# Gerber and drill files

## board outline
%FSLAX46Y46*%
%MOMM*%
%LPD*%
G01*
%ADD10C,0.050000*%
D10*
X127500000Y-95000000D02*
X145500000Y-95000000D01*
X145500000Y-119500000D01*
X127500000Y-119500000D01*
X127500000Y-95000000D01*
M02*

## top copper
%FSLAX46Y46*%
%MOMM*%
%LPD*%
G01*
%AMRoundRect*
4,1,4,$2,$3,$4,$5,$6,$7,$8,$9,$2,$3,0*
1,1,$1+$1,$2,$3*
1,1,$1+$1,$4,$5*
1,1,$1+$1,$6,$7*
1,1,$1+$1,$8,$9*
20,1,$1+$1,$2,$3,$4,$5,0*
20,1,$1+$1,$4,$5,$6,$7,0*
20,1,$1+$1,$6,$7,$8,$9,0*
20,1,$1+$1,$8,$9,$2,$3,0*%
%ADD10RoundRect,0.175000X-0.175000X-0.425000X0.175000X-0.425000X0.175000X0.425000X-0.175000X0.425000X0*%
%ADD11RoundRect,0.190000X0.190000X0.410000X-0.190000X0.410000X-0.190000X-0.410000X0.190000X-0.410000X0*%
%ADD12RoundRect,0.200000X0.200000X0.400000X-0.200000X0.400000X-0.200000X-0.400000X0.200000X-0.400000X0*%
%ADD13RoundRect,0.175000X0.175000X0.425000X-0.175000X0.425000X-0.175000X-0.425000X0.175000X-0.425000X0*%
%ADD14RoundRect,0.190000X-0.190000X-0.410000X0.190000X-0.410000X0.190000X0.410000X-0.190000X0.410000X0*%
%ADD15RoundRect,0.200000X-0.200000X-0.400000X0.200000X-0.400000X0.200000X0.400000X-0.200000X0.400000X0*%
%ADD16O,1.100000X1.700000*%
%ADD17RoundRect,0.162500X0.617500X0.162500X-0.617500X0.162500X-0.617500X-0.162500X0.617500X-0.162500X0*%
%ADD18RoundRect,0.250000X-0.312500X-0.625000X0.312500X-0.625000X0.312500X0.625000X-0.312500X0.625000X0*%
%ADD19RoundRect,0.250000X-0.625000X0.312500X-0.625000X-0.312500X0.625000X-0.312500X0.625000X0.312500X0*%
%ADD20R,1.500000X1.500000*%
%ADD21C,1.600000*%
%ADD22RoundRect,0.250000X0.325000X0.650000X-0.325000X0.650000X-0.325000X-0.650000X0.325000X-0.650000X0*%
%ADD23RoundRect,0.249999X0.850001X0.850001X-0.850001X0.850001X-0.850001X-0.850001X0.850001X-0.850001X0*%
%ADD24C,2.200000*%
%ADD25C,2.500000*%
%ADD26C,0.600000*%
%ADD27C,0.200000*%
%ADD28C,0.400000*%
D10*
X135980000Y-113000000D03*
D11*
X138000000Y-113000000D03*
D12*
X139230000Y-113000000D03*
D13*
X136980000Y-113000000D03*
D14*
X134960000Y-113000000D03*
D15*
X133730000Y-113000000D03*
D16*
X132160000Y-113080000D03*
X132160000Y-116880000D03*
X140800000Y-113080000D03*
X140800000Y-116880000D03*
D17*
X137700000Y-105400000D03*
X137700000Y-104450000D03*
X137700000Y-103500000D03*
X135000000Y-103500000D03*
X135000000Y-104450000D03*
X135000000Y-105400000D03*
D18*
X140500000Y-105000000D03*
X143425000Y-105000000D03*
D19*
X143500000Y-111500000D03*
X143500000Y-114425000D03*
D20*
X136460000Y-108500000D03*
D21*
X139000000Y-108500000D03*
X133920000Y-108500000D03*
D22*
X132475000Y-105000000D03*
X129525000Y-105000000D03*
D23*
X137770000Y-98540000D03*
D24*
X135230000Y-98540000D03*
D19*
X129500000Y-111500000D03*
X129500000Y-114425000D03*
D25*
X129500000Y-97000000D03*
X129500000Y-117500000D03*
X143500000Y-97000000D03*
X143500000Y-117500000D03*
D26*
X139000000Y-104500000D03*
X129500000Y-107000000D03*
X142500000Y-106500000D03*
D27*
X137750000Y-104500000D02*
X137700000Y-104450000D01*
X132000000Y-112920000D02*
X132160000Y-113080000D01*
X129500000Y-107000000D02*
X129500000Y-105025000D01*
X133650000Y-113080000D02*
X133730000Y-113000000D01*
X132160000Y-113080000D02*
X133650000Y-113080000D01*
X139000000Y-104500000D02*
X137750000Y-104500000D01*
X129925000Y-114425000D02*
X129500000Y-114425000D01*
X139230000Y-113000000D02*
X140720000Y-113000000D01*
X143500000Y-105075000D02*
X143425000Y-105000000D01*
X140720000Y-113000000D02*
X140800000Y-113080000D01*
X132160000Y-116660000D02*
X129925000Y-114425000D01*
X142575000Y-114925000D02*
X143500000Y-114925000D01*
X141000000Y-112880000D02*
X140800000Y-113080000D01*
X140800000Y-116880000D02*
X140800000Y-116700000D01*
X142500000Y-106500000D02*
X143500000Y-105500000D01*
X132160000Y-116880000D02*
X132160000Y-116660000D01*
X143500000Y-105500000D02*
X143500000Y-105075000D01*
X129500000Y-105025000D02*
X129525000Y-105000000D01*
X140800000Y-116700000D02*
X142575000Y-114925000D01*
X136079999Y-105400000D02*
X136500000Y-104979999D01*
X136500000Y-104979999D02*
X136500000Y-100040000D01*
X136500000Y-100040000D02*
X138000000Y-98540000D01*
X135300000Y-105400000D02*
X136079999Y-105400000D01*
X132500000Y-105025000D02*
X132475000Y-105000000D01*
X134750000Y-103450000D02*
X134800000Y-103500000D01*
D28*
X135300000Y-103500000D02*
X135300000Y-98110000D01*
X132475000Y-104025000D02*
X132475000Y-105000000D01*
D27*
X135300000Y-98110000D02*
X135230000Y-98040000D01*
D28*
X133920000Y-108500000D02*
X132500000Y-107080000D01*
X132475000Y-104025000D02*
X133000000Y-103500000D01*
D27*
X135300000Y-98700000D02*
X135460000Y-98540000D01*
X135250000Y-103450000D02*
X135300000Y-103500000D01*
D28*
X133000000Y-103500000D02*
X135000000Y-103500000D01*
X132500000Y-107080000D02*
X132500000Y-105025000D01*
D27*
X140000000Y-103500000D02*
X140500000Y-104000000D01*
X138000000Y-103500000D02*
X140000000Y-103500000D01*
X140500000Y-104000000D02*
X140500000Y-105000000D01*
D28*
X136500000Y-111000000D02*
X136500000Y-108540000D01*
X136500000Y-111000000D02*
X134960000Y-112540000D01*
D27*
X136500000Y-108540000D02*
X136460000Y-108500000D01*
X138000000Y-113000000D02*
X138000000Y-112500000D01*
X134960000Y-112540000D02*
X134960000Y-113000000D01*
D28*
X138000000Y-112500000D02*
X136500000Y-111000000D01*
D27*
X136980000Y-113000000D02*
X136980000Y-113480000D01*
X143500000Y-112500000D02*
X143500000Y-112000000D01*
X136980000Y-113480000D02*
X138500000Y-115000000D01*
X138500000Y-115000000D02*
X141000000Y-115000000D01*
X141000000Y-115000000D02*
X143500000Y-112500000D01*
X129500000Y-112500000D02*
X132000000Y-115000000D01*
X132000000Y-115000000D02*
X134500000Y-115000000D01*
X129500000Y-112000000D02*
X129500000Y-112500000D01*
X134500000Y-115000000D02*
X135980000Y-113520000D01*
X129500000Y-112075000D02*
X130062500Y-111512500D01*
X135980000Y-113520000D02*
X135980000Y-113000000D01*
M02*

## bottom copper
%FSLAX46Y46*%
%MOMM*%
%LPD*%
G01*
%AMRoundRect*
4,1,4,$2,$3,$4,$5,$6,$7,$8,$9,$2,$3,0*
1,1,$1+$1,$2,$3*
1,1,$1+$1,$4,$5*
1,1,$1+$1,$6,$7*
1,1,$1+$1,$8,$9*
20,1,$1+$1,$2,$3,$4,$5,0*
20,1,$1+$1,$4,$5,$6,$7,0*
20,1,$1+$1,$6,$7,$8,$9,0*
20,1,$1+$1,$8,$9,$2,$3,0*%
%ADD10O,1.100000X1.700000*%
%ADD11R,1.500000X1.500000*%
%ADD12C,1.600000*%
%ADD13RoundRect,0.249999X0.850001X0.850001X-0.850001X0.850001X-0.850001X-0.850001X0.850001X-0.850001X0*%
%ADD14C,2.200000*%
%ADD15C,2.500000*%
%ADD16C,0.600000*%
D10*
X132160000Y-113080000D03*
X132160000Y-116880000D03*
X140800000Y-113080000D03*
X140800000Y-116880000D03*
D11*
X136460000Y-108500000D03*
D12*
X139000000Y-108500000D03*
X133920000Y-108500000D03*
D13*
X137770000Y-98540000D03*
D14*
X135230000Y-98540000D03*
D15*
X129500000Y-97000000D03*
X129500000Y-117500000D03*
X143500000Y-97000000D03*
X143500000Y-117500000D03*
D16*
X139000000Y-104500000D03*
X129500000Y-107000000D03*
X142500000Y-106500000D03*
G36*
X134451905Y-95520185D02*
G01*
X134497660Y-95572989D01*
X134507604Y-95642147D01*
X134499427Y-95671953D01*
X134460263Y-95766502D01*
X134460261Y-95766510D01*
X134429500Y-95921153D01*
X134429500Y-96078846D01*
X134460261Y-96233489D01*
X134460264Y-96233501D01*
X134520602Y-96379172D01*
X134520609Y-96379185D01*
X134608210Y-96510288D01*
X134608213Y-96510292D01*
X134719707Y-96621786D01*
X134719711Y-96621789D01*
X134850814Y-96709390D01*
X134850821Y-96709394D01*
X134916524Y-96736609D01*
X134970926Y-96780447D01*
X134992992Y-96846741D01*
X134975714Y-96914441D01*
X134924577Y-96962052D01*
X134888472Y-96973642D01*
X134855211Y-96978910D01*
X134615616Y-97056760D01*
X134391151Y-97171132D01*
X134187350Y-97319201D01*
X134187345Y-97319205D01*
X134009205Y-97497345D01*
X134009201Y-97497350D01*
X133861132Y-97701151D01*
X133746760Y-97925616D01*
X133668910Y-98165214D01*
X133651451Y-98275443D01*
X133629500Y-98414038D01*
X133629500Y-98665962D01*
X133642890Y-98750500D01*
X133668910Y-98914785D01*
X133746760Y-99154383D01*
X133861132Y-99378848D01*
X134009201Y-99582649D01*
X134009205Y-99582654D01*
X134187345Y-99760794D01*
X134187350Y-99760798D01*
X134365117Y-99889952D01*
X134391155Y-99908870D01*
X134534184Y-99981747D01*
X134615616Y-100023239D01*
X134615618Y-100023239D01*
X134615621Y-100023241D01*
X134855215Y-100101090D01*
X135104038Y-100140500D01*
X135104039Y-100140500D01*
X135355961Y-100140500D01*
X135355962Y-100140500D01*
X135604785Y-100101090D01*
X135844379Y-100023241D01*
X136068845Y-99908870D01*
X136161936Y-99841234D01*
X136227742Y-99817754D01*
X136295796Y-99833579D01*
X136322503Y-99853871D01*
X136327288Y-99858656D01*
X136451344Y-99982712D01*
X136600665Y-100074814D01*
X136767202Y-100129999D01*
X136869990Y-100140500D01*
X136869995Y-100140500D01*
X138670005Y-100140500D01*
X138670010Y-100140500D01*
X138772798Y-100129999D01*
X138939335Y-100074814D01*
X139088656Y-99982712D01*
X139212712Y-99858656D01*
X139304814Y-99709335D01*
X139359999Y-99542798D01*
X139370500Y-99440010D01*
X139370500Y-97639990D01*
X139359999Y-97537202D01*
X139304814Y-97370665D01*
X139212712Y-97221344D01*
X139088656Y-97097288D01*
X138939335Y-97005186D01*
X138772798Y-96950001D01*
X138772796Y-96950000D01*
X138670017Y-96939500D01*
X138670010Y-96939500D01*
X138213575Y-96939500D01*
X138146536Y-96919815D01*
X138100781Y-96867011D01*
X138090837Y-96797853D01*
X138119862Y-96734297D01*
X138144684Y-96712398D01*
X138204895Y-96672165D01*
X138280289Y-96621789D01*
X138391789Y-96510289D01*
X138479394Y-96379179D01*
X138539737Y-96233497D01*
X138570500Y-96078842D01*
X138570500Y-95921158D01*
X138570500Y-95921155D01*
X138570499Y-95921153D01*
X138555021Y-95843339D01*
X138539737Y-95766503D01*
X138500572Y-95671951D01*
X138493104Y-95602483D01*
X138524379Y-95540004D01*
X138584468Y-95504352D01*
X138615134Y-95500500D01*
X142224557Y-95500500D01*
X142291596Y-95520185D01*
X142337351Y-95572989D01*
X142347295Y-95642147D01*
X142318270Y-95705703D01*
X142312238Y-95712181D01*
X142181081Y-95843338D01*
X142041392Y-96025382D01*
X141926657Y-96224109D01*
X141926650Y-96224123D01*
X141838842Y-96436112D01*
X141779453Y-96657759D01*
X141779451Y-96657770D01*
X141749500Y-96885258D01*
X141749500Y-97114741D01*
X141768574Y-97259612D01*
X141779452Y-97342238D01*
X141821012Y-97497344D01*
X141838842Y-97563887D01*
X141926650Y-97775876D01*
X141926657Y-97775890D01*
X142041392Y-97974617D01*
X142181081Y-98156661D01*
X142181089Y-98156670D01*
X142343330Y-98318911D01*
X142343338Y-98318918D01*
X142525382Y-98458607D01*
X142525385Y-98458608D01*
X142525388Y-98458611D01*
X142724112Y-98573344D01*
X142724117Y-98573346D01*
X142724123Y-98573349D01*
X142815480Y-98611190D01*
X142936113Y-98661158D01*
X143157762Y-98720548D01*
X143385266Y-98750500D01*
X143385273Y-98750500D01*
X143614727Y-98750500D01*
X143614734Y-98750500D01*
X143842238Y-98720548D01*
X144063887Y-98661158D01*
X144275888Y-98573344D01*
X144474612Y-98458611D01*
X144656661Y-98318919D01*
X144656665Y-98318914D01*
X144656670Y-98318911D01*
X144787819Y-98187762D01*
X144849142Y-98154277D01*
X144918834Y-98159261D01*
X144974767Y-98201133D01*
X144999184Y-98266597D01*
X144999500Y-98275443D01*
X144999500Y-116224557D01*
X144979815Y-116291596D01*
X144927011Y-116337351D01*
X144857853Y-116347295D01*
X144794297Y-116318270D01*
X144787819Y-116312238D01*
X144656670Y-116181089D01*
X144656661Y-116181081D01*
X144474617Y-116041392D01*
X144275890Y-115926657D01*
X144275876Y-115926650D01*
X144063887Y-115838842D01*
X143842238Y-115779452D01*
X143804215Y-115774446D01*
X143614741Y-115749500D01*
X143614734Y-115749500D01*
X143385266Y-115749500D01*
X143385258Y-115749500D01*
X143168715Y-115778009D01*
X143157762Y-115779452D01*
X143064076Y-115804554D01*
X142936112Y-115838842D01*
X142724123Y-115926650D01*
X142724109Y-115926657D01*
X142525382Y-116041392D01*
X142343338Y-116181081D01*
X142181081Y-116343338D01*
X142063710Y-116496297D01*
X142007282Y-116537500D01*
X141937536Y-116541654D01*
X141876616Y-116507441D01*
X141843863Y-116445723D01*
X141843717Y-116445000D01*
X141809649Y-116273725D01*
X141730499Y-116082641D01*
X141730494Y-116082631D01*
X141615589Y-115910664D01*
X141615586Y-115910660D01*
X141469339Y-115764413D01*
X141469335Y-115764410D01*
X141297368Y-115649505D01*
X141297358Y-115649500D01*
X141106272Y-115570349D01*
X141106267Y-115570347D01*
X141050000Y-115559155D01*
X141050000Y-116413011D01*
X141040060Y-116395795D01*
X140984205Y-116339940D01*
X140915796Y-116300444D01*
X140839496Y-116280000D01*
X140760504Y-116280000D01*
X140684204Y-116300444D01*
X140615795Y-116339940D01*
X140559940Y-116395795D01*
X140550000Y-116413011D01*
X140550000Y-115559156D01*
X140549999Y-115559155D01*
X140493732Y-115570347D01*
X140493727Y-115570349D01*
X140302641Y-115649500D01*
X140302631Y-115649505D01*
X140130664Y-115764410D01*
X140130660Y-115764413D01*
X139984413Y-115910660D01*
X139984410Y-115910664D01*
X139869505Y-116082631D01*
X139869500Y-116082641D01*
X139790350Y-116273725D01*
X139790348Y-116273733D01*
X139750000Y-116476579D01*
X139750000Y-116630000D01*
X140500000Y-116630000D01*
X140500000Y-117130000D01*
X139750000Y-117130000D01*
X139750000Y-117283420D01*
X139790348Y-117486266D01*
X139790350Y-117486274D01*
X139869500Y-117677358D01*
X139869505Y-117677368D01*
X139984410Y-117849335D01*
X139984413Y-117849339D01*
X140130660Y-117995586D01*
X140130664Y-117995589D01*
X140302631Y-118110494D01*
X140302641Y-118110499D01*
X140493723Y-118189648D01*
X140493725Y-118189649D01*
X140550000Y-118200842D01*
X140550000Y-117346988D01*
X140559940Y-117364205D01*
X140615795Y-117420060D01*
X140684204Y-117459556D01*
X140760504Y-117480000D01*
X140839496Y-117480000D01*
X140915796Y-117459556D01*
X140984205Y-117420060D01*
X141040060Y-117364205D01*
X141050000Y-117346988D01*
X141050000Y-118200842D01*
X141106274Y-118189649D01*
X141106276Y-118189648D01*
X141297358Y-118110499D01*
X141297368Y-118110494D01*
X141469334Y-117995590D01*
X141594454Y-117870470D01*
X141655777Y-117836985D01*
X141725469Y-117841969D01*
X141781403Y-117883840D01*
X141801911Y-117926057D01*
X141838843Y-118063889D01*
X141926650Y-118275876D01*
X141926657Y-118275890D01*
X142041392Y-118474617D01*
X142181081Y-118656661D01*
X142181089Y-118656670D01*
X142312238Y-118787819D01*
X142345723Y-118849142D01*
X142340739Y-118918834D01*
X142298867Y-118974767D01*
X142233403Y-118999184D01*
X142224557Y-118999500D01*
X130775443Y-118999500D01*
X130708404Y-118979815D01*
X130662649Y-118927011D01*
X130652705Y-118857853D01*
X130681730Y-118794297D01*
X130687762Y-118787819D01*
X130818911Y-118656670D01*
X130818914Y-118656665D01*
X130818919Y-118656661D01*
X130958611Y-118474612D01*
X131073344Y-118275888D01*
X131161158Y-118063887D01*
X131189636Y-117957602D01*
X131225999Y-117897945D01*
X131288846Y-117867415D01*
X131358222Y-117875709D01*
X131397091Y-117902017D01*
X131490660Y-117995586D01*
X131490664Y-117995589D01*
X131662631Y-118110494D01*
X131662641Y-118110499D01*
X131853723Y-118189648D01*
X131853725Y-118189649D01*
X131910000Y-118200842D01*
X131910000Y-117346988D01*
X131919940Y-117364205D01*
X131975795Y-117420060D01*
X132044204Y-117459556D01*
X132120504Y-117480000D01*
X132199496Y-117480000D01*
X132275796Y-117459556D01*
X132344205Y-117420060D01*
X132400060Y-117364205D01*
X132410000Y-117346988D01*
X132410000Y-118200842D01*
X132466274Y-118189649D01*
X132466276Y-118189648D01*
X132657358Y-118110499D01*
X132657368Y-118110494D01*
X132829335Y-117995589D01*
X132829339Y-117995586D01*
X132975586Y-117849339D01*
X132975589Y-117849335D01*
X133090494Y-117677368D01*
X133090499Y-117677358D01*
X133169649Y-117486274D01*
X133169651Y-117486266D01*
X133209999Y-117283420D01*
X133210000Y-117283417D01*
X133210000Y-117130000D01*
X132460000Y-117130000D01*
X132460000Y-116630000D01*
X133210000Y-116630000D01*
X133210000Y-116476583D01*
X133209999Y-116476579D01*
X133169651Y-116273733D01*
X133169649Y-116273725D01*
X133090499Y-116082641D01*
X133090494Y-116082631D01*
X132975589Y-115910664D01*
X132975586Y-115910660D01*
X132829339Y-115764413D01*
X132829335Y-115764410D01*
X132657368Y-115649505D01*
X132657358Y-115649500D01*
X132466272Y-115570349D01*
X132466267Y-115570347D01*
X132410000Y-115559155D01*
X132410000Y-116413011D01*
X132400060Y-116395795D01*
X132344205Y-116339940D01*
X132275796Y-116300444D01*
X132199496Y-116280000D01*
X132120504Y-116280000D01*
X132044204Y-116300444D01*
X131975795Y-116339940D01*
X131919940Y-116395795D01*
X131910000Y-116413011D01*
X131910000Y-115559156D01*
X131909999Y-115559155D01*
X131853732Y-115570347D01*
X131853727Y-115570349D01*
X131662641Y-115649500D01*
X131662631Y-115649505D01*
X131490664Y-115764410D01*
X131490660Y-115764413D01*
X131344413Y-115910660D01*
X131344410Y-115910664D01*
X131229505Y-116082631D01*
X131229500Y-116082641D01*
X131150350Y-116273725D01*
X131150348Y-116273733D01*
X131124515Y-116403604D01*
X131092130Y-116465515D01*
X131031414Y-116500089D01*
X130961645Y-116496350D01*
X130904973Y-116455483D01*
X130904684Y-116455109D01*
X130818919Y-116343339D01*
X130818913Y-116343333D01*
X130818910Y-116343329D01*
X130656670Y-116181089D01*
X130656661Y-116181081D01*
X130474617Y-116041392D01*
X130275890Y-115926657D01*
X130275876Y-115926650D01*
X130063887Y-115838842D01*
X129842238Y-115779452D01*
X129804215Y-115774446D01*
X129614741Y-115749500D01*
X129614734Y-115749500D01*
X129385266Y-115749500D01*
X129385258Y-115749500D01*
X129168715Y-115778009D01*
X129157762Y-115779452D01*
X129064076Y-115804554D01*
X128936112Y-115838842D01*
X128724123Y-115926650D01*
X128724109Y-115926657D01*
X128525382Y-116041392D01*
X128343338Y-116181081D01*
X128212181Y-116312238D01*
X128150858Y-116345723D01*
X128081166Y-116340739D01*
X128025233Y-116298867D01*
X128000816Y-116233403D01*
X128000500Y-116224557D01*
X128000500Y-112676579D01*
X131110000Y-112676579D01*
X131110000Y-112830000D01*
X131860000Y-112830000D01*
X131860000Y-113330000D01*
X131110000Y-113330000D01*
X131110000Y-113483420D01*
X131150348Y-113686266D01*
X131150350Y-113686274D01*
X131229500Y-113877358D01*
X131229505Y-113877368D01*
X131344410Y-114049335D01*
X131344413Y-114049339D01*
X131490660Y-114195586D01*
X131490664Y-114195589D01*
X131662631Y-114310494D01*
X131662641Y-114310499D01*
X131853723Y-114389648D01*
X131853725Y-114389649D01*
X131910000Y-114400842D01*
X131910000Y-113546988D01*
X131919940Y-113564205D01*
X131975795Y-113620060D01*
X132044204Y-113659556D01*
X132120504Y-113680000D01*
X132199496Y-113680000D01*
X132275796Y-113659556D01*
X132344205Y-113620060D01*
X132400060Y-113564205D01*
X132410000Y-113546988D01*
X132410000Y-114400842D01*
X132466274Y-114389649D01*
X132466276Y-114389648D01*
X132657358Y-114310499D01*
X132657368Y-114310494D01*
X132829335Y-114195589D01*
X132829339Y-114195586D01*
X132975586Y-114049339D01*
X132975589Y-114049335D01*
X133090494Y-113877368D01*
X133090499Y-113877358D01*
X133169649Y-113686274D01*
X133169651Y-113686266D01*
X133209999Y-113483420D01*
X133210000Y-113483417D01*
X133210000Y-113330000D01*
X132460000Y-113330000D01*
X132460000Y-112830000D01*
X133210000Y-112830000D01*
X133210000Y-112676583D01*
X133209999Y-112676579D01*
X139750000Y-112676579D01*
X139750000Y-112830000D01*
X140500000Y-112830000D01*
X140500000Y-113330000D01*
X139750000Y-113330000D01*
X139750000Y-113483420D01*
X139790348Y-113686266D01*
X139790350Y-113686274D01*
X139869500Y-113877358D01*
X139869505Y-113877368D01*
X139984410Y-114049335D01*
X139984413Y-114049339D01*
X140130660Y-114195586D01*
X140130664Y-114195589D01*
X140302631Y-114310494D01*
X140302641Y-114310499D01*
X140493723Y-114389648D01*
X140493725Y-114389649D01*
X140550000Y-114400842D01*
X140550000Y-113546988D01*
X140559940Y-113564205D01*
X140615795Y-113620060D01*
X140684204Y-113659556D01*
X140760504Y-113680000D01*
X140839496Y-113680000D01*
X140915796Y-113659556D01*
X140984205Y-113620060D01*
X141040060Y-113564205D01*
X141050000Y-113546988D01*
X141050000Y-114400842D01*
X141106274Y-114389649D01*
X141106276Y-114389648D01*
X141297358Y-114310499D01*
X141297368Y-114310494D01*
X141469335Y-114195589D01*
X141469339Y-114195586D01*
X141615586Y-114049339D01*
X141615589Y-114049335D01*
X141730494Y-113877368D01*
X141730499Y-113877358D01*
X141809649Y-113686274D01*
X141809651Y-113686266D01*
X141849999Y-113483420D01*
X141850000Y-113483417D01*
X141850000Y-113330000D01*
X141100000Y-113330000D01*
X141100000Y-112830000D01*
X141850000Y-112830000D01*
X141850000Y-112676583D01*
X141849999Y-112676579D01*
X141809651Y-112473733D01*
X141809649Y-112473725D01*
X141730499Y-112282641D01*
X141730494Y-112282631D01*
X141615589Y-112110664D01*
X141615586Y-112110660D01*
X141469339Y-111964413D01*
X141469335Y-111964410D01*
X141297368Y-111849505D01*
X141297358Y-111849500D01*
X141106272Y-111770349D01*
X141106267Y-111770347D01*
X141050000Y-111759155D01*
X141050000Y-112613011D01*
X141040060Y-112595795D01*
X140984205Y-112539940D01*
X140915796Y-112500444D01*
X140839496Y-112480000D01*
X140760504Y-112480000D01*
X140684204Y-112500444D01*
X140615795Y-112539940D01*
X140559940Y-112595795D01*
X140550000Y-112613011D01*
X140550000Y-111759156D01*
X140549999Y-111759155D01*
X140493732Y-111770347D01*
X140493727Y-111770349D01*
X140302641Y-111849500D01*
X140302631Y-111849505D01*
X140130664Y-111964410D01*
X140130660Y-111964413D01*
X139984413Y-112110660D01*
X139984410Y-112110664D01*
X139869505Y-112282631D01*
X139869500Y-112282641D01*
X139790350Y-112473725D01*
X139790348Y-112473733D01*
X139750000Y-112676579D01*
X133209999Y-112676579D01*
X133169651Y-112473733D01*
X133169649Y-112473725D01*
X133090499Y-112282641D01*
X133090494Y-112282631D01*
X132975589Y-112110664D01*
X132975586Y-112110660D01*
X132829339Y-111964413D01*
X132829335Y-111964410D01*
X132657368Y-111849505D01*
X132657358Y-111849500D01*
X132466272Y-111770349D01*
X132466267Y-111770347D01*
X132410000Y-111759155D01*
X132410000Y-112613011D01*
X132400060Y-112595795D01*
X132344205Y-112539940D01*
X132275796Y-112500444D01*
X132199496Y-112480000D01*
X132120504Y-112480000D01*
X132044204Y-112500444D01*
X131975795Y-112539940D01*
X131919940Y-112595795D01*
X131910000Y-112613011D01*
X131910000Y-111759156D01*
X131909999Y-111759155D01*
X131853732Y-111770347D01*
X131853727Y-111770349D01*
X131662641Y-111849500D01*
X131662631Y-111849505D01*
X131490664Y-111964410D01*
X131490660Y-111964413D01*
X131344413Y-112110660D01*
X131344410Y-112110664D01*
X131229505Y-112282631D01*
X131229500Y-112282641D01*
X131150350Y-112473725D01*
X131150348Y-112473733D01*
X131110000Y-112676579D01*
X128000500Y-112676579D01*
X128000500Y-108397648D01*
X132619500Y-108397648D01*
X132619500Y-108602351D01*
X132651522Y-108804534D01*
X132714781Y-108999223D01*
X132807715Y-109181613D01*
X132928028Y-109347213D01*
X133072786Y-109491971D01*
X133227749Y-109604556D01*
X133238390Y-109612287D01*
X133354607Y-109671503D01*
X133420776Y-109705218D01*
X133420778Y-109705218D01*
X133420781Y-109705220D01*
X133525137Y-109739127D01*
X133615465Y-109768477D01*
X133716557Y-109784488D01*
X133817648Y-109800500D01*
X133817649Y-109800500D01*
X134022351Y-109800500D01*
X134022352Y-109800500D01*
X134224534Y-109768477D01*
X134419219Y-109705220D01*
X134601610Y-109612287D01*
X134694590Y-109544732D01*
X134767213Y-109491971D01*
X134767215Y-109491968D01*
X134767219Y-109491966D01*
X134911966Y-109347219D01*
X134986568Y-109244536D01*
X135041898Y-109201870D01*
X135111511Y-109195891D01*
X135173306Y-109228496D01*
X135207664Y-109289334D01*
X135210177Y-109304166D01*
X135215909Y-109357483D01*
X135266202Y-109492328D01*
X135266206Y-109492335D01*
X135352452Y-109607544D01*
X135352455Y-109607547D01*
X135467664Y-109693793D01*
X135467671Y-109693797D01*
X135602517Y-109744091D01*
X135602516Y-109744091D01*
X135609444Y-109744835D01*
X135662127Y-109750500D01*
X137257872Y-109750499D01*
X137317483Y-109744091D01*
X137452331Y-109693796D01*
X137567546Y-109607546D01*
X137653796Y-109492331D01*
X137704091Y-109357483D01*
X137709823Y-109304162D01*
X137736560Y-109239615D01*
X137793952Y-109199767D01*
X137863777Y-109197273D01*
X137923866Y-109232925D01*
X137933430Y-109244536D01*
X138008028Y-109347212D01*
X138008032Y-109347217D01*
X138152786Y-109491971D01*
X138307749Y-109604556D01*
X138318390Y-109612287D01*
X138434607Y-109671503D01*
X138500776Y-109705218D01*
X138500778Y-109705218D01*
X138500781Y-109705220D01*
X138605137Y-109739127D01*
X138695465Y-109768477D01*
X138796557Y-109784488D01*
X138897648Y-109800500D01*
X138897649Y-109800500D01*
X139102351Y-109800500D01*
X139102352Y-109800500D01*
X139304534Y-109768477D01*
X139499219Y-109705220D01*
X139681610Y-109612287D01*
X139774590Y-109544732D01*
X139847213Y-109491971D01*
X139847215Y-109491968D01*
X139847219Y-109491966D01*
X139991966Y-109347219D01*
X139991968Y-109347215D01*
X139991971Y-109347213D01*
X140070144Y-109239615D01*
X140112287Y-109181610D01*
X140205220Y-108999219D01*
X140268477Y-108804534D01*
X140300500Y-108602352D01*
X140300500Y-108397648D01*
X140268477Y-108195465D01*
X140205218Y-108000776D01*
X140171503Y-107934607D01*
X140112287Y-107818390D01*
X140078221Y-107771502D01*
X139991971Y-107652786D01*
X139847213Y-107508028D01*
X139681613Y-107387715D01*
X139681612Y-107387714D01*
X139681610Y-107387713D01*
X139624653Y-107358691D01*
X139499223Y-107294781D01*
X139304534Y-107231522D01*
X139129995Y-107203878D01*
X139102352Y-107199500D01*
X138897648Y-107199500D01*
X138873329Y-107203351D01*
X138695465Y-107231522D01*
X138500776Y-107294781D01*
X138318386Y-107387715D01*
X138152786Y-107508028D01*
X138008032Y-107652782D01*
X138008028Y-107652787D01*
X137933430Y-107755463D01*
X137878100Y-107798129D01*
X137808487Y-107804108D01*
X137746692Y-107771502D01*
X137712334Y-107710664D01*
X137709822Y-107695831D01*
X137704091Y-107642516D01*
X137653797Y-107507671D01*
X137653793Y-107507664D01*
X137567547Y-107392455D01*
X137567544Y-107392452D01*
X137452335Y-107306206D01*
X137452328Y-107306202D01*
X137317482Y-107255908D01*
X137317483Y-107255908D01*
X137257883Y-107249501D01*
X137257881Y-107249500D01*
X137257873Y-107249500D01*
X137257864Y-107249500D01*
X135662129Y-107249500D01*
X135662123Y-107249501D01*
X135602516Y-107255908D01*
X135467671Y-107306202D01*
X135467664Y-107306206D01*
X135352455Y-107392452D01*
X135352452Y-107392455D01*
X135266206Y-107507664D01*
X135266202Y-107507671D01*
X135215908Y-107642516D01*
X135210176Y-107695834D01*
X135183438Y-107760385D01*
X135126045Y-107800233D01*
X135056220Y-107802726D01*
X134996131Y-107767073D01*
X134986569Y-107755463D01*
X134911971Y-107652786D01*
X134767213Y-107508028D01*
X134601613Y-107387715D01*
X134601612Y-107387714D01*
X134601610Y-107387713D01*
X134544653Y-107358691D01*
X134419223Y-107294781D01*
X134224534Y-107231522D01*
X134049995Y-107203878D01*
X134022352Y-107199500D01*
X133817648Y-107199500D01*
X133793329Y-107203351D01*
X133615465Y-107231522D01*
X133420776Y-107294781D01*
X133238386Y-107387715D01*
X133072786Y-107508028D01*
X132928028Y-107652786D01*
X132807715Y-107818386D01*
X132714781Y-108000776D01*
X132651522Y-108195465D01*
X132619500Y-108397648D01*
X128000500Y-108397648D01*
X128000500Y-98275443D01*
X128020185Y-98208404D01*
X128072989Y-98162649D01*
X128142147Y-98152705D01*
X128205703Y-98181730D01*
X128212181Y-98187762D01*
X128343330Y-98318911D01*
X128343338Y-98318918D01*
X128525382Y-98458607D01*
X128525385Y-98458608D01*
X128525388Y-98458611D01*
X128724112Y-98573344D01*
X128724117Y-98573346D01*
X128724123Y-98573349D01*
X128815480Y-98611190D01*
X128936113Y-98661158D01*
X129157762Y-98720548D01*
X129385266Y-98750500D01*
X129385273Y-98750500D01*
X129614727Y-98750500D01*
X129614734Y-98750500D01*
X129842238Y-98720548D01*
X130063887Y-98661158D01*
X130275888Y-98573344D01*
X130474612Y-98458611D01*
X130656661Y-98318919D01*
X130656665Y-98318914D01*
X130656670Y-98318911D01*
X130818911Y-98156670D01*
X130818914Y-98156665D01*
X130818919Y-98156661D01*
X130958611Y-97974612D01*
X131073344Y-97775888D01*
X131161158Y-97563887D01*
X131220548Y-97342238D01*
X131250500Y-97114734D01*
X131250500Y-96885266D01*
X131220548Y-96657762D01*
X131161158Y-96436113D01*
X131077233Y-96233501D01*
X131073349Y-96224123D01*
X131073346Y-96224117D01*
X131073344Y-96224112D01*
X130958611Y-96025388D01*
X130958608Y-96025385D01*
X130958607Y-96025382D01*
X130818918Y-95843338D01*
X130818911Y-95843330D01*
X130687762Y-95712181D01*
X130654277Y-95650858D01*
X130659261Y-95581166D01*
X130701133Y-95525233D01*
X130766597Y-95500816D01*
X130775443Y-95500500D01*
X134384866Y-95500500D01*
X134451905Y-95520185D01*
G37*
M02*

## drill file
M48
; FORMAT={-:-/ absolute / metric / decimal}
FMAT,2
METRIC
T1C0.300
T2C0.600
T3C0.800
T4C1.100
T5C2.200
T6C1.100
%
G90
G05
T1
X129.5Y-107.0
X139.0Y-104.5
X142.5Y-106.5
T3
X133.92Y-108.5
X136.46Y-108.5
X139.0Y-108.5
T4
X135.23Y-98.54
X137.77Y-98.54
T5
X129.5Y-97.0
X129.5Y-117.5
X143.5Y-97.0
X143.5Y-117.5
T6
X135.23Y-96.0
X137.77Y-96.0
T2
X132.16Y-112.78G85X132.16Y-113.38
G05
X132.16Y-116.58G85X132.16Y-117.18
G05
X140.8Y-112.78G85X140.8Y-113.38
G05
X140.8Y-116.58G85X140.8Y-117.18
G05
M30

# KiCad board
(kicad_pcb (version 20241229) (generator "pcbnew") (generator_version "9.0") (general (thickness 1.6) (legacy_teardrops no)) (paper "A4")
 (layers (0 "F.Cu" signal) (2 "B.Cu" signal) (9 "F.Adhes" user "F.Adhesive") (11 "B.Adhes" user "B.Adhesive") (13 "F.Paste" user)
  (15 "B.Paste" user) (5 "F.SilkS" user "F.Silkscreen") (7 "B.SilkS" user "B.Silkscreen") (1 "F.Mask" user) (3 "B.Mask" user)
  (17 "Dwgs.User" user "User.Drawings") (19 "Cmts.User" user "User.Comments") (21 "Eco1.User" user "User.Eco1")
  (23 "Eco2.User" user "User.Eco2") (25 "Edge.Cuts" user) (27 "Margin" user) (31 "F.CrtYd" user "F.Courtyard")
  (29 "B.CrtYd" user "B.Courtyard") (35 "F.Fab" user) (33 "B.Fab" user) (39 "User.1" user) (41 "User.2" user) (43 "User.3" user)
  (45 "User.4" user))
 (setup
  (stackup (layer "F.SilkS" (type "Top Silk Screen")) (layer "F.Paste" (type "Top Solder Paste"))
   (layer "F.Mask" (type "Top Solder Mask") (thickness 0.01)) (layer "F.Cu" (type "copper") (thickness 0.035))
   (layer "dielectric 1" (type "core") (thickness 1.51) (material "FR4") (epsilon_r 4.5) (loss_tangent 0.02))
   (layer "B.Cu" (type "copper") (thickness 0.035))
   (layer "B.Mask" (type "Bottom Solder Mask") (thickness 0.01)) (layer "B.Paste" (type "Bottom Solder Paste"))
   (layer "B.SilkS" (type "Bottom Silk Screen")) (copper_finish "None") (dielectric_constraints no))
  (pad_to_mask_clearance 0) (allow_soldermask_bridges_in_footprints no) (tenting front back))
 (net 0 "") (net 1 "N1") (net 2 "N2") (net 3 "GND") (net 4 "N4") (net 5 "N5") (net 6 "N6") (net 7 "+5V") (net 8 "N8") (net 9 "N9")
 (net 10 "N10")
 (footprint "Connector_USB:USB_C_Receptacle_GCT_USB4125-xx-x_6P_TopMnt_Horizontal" (layer "F.Cu") (at 136.48 116.08)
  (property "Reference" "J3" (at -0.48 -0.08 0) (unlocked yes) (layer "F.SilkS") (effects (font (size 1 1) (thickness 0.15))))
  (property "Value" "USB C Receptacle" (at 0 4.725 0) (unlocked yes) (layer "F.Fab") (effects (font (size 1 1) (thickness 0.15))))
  (pad "A5" smd roundrect (at -0.5 -3.08) (size 0.7 1.2) (layers "F.Cu" "F.Mask" "F.Paste") (roundrect_rratio 0.25) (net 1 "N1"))
  (pad "A9" smd roundrect (at 1.52 -3.08 180) (size 0.76 1.2) (layers "F.Cu" "F.Mask" "F.Paste") (roundrect_rratio 0.25) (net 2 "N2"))
  (pad "A12" smd roundrect (at 2.75 -3.08 180) (size 0.8 1.2) (layers "F.Cu" "F.Mask" "F.Paste") (roundrect_rratio 0.25) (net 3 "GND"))
  (pad "B5" smd roundrect (at 0.5 -3.08 180) (size 0.7 1.2) (layers "F.Cu" "F.Mask" "F.Paste") (roundrect_rratio 0.25) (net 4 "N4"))
  (pad "B9" smd roundrect (at -1.52 -3.08) (size 0.76 1.2) (layers "F.Cu" "F.Mask" "F.Paste") (roundrect_rratio 0.25) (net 2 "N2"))
  (pad "B12" smd roundrect (at -2.75 -3.08) (size 0.8 1.2) (layers "F.Cu" "F.Mask" "F.Paste") (roundrect_rratio 0.25) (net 3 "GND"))
  (pad "S1" thru_hole oval (at -4.32 -3) (size 1.1 1.7) (drill oval 0.6 1.2) (layers "*.Cu" "*.Mask" "F.Paste") (remove_unused_layers no)
   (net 3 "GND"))
  (pad "S1" thru_hole oval (at -4.32 0.8) (size 1.1 1.7) (drill oval 0.6 1.2) (layers "*.Cu" "*.Mask" "F.Paste") (remove_unused_layers no)
   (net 3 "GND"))
  (pad "S1" thru_hole oval (at 4.32 -3) (size 1.1 1.7) (drill oval 0.6 1.2) (layers "*.Cu" "*.Mask" "F.Paste") (remove_unused_layers no)
   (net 3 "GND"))
  (pad "S1" thru_hole oval (at 4.32 0.8) (size 1.1 1.7) (drill oval 0.6 1.2) (layers "*.Cu" "*.Mask" "F.Paste") (remove_unused_layers no)
   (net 3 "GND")))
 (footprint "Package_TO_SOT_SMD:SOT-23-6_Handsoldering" (layer "F.Cu") (at 136.35 104.45 180)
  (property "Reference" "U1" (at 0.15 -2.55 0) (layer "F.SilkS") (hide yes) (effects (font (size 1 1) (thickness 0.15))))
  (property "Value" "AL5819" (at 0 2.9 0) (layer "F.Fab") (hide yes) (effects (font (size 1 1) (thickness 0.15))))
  (pad "1" smd roundrect (at -1.35 -0.95 180) (size 1.56 0.65) (layers "F.Cu" "F.Mask" "F.Paste") (roundrect_rratio 0.25) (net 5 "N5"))
  (pad "2" smd roundrect (at -1.35 0 180) (size 1.56 0.65) (layers "F.Cu" "F.Mask" "F.Paste") (roundrect_rratio 0.25) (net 3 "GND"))
  (pad "3" smd roundrect (at -1.35 0.95 180) (size 1.56 0.65) (layers "F.Cu" "F.Mask" "F.Paste") (roundrect_rratio 0.25) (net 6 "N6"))
  (pad "4" smd roundrect (at 1.35 0.95 180) (size 1.56 0.65) (layers "F.Cu" "F.Mask" "F.Paste") (roundrect_rratio 0.25) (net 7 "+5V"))
  (pad "5" smd roundrect (at 1.35 0 180) (size 1.56 0.65) (layers "F.Cu" "F.Mask" "F.Paste") (roundrect_rratio 0.25) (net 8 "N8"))
  (pad "6" smd roundrect (at 1.35 -0.95 180) (size 1.56 0.65) (layers "F.Cu" "F.Mask" "F.Paste") (roundrect_rratio 0.25) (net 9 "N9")))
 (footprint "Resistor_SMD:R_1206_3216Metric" (layer "F.Cu") (at 141.9625 105)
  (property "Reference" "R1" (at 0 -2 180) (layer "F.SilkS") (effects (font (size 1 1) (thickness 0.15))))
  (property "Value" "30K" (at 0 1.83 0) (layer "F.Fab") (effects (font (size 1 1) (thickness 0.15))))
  (pad "1" smd roundrect (at -1.4625 0) (size 1.125 1.75) (layers "F.Cu" "F.Mask" "F.Paste") (roundrect_rratio 0.222222) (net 6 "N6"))
  (pad "2" smd roundrect (at 1.4625 0) (size 1.125 1.75) (layers "F.Cu" "F.Mask" "F.Paste") (roundrect_rratio 0.222222) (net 3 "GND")))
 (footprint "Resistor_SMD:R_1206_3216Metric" (layer "F.Cu") (at 143.5 112.9625 -90)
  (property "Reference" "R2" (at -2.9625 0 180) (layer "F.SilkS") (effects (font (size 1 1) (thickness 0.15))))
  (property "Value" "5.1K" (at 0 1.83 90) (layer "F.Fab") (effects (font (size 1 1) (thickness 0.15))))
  (pad "1" smd roundrect (at -1.4625 0 270) (size 1.125 1.75) (layers "F.Cu" "F.Mask" "F.Paste") (roundrect_rratio 0.222222) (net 4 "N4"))
  (pad "2" smd roundrect (at 1.4625 0 270) (size 1.125 1.75) (layers "F.Cu" "F.Mask" "F.Paste") (roundrect_rratio 0.222222) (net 3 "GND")))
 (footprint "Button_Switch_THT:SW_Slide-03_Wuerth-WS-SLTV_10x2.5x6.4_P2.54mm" (layer "F.Cu") (at 136.46 108.5 180)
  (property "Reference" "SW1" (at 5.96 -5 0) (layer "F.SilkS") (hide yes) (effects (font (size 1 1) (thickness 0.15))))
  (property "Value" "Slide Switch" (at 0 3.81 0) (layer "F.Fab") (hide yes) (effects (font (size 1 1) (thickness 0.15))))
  (pad "1" thru_hole rect (at 0 0 180) (size 1.5 1.5) (drill 0.8) (layers "*.Cu" "*.Mask") (remove_unused_layers no) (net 2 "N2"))
  (pad "2" thru_hole circle (at -2.54 0 180) (size 1.6 1.6) (drill 0.8) (layers "*.Cu" "*.Mask") (remove_unused_layers no) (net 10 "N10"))
  (pad "3" thru_hole circle (at 2.54 0 180) (size 1.6 1.6) (drill 0.8) (layers "*.Cu" "*.Mask") (remove_unused_layers no) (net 7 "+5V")))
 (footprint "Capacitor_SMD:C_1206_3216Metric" (layer "F.Cu") (at 131 105 180)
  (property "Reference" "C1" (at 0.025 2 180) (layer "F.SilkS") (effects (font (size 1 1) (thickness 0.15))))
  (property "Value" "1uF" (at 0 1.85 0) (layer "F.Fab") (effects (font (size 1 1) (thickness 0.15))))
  (pad "1" smd roundrect (at -1.475 0 180) (size 1.15 1.8) (layers "F.Cu" "F.Mask" "F.Paste") (roundrect_rratio 0.217391) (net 7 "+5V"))
  (pad "2" smd roundrect (at 1.475 0 180) (size 1.15 1.8) (layers "F.Cu" "F.Mask" "F.Paste") (roundrect_rratio 0.217391) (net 3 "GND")))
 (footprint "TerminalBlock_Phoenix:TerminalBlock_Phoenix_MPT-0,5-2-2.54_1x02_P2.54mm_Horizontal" (layer "F.Cu") (at 137.77 98.54 180)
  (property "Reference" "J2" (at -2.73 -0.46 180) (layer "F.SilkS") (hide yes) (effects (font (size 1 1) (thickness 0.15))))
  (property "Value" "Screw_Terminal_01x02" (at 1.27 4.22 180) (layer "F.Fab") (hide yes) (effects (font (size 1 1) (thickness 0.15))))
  (pad "" np_thru_hole circle (at 0 2.54 180) (size 1.1 1.1) (drill 1.1) (layers "*.Cu" "*.Mask"))
  (pad "" np_thru_hole circle (at 2.54 2.54 180) (size 1.1 1.1) (drill 1.1) (layers "*.Cu" "*.Mask"))
  (pad "1" thru_hole roundrect (at 0 0 180) (size 2.2 2.2) (drill 1.1) (layers "*.Cu" "*.Mask") (remove_unused_layers no)
   (roundrect_rratio 0.113636) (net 9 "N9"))
  (pad "2" thru_hole circle (at 2.54 0 180) (size 2.2 2.2) (drill 1.1) (layers "*.Cu" "*.Mask") (remove_unused_layers no) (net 7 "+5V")))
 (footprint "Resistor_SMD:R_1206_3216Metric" (layer "F.Cu") (at 129.5 112.9625 -90)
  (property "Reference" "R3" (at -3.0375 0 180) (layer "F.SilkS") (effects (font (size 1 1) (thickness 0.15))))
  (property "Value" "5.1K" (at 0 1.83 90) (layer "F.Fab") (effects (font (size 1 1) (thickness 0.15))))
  (pad "1" smd roundrect (at -1.4625 0 270) (size 1.125 1.75) (layers "F.Cu" "F.Mask" "F.Paste") (roundrect_rratio 0.222222) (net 1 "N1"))
  (pad "2" smd roundrect (at 1.4625 0 270) (size 1.125 1.75) (layers "F.Cu" "F.Mask" "F.Paste") (roundrect_rratio 0.222222) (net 3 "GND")))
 (gr_rect (start 127.5 95) (end 145.5 119.5) (stroke (width 0.05) (type default)) (fill no) (layer "Edge.Cuts"))
 (via (at 129.5 97) (size 2.5) (drill 2.2) (layers "F.Cu" "B.Cu") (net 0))
 (via (at 129.5 117.5) (size 2.5) (drill 2.2) (layers "F.Cu" "B.Cu") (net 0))
 (via (at 143.5 97) (size 2.5) (drill 2.2) (layers "F.Cu" "B.Cu") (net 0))
 (via (at 143.5 117.5) (size 2.5) (drill 2.2) (layers "F.Cu" "B.Cu") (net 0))
 (segment (start 137.75 104.5) (end 137.7 104.45) (width 0.2) (layer "F.Cu") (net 3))
 (segment (start 132 112.92) (end 132.16 113.08) (width 0.2) (layer "F.Cu") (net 3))
 (segment (start 129.5 107) (end 129.5 105.025) (width 0.2) (layer "F.Cu") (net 3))
 (segment (start 133.65 113.08) (end 133.73 113) (width 0.2) (layer "F.Cu") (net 3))
 (segment (start 132.16 113.08) (end 133.65 113.08) (width 0.2) (layer "F.Cu") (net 3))
 (segment (start 139 104.5) (end 137.75 104.5) (width 0.2) (layer "F.Cu") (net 3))
 (segment (start 129.925 114.425) (end 129.5 114.425) (width 0.2) (layer "F.Cu") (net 3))
 (segment (start 139.23 113) (end 140.72 113) (width 0.2) (layer "F.Cu") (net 3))
 (segment (start 143.5 105.075) (end 143.425 105) (width 0.2) (layer "F.Cu") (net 3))
 (segment (start 140.72 113) (end 140.8 113.08) (width 0.2) (layer "F.Cu") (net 3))
 (segment (start 132.16 116.66) (end 129.925 114.425) (width 0.2) (layer "F.Cu") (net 3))
 (segment (start 142.575 114.925) (end 143.5 114.925) (width 0.2) (layer "F.Cu") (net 3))
 (segment (start 141 112.88) (end 140.8 113.08) (width 0.2) (layer "F.Cu") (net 3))
 (segment (start 140.8 116.88) (end 140.8 116.7) (width 0.2) (layer "F.Cu") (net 3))
 (segment (start 142.5 106.5) (end 143.5 105.5) (width 0.2) (layer "F.Cu") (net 3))
 (segment (start 132.16 116.88) (end 132.16 116.66) (width 0.2) (layer "F.Cu") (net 3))
 (segment (start 143.5 105.5) (end 143.5 105.075) (width 0.2) (layer "F.Cu") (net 3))
 (segment (start 129.5 105.025) (end 129.525 105) (width 0.2) (layer "F.Cu") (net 3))
 (segment (start 140.8 116.7) (end 142.575 114.925) (width 0.2) (layer "F.Cu") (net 3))
 (via (at 139 104.5) (size 0.6) (drill 0.3) (layers "F.Cu" "B.Cu") (free yes) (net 3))
 (via (at 129.5 107) (size 0.6) (drill 0.3) (layers "F.Cu" "B.Cu") (free yes) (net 3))
 (via (at 142.5 106.5) (size 0.6) (drill 0.3) (layers "F.Cu" "B.Cu") (free yes) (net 3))
 (segment (start 136.079999 105.4) (end 136.5 104.979999) (width 0.2) (layer "F.Cu") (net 9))
 (segment (start 136.5 104.979999) (end 136.5 100.04) (width 0.2) (layer "F.Cu") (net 9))
 (segment (start 136.5 100.04) (end 138 98.54) (width 0.2) (layer "F.Cu") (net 9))
 (segment (start 135.3 105.4) (end 136.079999 105.4) (width 0.2) (layer "F.Cu") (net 9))
 (segment (start 132.5 105.025) (end 132.475 105) (width 0.2) (layer "F.Cu") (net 7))
 (segment (start 134.75 103.45) (end 134.8 103.5) (width 0.2) (layer "F.Cu") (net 7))
 (segment (start 135.3 103.5) (end 135.3 98.11) (width 0.4) (layer "F.Cu") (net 7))
 (segment (start 132.475 104.025) (end 132.475 105) (width 0.4) (layer "F.Cu") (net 7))
 (segment (start 135.3 98.11) (end 135.23 98.04) (width 0.2) (layer "F.Cu") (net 7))
 (segment (start 133.92 108.5) (end 132.5 107.08) (width 0.4) (layer "F.Cu") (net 7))
 (segment (start 132.475 104.025) (end 133 103.5) (width 0.4) (layer "F.Cu") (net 7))
 (segment (start 135.3 98.7) (end 135.46 98.54) (width 0.2) (layer "F.Cu") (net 7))
 (segment (start 135.25 103.45) (end 135.3 103.5) (width 0.2) (layer "F.Cu") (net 7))
 (segment (start 133 103.5) (end 135 103.5) (width 0.4) (layer "F.Cu") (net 7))
 (segment (start 132.5 107.08) (end 132.5 105.025) (width 0.4) (layer "F.Cu") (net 7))
 (segment (start 140 103.5) (end 140.5 104) (width 0.2) (layer "F.Cu") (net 6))
 (segment (start 138 103.5) (end 140 103.5) (width 0.2) (layer "F.Cu") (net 6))
 (segment (start 140.5 104) (end 140.5 105) (width 0.2) (layer "F.Cu") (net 6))
 (segment (start 136.5 111) (end 136.5 108.54) (width 0.4) (layer "F.Cu") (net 2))
 (segment (start 136.5 111) (end 134.96 112.54) (width 0.4) (layer "F.Cu") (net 2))
 (segment (start 136.5 108.54) (end 136.46 108.5) (width 0.2) (layer "F.Cu") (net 2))
 (segment (start 138 113) (end 138 112.5) (width 0.2) (layer "F.Cu") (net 2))
 (segment (start 134.96 112.54) (end 134.96 113) (width 0.2) (layer "F.Cu") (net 2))
 (segment (start 138 112.5) (end 136.5 111) (width 0.4) (layer "F.Cu") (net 2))
 (segment (start 136.98 113) (end 136.98 113.48) (width 0.2) (layer "F.Cu") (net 4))
 (segment (start 143.5 112.5) (end 143.5 112) (width 0.2) (layer "F.Cu") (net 4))
 (segment (start 136.98 113.48) (end 138.5 115) (width 0.2) (layer "F.Cu") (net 4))
 (segment (start 138.5 115) (end 141 115) (width 0.2) (layer "F.Cu") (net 4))
 (segment (start 141 115) (end 143.5 112.5) (width 0.2) (layer "F.Cu") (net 4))
 (segment (start 129.5 112.5) (end 132 115) (width 0.2) (layer "F.Cu") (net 1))
 (segment (start 132 115) (end 134.5 115) (width 0.2) (layer "F.Cu") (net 1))
 (segment (start 129.5 112) (end 129.5 112.5) (width 0.2) (layer "F.Cu") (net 1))
 (segment (start 134.5 115) (end 135.98 113.52) (width 0.2) (layer "F.Cu") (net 1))
 (segment (start 129.5 112.075) (end 130.0625 111.5125) (width 0.2) (layer "F.Cu") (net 1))
 (segment (start 135.98 113.52) (end 135.98 113) (width 0.2) (layer "F.Cu") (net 1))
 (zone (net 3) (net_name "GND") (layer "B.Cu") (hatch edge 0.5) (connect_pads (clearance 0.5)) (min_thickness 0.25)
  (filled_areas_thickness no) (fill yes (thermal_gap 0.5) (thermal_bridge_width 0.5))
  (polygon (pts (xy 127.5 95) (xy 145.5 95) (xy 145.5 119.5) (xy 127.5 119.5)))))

